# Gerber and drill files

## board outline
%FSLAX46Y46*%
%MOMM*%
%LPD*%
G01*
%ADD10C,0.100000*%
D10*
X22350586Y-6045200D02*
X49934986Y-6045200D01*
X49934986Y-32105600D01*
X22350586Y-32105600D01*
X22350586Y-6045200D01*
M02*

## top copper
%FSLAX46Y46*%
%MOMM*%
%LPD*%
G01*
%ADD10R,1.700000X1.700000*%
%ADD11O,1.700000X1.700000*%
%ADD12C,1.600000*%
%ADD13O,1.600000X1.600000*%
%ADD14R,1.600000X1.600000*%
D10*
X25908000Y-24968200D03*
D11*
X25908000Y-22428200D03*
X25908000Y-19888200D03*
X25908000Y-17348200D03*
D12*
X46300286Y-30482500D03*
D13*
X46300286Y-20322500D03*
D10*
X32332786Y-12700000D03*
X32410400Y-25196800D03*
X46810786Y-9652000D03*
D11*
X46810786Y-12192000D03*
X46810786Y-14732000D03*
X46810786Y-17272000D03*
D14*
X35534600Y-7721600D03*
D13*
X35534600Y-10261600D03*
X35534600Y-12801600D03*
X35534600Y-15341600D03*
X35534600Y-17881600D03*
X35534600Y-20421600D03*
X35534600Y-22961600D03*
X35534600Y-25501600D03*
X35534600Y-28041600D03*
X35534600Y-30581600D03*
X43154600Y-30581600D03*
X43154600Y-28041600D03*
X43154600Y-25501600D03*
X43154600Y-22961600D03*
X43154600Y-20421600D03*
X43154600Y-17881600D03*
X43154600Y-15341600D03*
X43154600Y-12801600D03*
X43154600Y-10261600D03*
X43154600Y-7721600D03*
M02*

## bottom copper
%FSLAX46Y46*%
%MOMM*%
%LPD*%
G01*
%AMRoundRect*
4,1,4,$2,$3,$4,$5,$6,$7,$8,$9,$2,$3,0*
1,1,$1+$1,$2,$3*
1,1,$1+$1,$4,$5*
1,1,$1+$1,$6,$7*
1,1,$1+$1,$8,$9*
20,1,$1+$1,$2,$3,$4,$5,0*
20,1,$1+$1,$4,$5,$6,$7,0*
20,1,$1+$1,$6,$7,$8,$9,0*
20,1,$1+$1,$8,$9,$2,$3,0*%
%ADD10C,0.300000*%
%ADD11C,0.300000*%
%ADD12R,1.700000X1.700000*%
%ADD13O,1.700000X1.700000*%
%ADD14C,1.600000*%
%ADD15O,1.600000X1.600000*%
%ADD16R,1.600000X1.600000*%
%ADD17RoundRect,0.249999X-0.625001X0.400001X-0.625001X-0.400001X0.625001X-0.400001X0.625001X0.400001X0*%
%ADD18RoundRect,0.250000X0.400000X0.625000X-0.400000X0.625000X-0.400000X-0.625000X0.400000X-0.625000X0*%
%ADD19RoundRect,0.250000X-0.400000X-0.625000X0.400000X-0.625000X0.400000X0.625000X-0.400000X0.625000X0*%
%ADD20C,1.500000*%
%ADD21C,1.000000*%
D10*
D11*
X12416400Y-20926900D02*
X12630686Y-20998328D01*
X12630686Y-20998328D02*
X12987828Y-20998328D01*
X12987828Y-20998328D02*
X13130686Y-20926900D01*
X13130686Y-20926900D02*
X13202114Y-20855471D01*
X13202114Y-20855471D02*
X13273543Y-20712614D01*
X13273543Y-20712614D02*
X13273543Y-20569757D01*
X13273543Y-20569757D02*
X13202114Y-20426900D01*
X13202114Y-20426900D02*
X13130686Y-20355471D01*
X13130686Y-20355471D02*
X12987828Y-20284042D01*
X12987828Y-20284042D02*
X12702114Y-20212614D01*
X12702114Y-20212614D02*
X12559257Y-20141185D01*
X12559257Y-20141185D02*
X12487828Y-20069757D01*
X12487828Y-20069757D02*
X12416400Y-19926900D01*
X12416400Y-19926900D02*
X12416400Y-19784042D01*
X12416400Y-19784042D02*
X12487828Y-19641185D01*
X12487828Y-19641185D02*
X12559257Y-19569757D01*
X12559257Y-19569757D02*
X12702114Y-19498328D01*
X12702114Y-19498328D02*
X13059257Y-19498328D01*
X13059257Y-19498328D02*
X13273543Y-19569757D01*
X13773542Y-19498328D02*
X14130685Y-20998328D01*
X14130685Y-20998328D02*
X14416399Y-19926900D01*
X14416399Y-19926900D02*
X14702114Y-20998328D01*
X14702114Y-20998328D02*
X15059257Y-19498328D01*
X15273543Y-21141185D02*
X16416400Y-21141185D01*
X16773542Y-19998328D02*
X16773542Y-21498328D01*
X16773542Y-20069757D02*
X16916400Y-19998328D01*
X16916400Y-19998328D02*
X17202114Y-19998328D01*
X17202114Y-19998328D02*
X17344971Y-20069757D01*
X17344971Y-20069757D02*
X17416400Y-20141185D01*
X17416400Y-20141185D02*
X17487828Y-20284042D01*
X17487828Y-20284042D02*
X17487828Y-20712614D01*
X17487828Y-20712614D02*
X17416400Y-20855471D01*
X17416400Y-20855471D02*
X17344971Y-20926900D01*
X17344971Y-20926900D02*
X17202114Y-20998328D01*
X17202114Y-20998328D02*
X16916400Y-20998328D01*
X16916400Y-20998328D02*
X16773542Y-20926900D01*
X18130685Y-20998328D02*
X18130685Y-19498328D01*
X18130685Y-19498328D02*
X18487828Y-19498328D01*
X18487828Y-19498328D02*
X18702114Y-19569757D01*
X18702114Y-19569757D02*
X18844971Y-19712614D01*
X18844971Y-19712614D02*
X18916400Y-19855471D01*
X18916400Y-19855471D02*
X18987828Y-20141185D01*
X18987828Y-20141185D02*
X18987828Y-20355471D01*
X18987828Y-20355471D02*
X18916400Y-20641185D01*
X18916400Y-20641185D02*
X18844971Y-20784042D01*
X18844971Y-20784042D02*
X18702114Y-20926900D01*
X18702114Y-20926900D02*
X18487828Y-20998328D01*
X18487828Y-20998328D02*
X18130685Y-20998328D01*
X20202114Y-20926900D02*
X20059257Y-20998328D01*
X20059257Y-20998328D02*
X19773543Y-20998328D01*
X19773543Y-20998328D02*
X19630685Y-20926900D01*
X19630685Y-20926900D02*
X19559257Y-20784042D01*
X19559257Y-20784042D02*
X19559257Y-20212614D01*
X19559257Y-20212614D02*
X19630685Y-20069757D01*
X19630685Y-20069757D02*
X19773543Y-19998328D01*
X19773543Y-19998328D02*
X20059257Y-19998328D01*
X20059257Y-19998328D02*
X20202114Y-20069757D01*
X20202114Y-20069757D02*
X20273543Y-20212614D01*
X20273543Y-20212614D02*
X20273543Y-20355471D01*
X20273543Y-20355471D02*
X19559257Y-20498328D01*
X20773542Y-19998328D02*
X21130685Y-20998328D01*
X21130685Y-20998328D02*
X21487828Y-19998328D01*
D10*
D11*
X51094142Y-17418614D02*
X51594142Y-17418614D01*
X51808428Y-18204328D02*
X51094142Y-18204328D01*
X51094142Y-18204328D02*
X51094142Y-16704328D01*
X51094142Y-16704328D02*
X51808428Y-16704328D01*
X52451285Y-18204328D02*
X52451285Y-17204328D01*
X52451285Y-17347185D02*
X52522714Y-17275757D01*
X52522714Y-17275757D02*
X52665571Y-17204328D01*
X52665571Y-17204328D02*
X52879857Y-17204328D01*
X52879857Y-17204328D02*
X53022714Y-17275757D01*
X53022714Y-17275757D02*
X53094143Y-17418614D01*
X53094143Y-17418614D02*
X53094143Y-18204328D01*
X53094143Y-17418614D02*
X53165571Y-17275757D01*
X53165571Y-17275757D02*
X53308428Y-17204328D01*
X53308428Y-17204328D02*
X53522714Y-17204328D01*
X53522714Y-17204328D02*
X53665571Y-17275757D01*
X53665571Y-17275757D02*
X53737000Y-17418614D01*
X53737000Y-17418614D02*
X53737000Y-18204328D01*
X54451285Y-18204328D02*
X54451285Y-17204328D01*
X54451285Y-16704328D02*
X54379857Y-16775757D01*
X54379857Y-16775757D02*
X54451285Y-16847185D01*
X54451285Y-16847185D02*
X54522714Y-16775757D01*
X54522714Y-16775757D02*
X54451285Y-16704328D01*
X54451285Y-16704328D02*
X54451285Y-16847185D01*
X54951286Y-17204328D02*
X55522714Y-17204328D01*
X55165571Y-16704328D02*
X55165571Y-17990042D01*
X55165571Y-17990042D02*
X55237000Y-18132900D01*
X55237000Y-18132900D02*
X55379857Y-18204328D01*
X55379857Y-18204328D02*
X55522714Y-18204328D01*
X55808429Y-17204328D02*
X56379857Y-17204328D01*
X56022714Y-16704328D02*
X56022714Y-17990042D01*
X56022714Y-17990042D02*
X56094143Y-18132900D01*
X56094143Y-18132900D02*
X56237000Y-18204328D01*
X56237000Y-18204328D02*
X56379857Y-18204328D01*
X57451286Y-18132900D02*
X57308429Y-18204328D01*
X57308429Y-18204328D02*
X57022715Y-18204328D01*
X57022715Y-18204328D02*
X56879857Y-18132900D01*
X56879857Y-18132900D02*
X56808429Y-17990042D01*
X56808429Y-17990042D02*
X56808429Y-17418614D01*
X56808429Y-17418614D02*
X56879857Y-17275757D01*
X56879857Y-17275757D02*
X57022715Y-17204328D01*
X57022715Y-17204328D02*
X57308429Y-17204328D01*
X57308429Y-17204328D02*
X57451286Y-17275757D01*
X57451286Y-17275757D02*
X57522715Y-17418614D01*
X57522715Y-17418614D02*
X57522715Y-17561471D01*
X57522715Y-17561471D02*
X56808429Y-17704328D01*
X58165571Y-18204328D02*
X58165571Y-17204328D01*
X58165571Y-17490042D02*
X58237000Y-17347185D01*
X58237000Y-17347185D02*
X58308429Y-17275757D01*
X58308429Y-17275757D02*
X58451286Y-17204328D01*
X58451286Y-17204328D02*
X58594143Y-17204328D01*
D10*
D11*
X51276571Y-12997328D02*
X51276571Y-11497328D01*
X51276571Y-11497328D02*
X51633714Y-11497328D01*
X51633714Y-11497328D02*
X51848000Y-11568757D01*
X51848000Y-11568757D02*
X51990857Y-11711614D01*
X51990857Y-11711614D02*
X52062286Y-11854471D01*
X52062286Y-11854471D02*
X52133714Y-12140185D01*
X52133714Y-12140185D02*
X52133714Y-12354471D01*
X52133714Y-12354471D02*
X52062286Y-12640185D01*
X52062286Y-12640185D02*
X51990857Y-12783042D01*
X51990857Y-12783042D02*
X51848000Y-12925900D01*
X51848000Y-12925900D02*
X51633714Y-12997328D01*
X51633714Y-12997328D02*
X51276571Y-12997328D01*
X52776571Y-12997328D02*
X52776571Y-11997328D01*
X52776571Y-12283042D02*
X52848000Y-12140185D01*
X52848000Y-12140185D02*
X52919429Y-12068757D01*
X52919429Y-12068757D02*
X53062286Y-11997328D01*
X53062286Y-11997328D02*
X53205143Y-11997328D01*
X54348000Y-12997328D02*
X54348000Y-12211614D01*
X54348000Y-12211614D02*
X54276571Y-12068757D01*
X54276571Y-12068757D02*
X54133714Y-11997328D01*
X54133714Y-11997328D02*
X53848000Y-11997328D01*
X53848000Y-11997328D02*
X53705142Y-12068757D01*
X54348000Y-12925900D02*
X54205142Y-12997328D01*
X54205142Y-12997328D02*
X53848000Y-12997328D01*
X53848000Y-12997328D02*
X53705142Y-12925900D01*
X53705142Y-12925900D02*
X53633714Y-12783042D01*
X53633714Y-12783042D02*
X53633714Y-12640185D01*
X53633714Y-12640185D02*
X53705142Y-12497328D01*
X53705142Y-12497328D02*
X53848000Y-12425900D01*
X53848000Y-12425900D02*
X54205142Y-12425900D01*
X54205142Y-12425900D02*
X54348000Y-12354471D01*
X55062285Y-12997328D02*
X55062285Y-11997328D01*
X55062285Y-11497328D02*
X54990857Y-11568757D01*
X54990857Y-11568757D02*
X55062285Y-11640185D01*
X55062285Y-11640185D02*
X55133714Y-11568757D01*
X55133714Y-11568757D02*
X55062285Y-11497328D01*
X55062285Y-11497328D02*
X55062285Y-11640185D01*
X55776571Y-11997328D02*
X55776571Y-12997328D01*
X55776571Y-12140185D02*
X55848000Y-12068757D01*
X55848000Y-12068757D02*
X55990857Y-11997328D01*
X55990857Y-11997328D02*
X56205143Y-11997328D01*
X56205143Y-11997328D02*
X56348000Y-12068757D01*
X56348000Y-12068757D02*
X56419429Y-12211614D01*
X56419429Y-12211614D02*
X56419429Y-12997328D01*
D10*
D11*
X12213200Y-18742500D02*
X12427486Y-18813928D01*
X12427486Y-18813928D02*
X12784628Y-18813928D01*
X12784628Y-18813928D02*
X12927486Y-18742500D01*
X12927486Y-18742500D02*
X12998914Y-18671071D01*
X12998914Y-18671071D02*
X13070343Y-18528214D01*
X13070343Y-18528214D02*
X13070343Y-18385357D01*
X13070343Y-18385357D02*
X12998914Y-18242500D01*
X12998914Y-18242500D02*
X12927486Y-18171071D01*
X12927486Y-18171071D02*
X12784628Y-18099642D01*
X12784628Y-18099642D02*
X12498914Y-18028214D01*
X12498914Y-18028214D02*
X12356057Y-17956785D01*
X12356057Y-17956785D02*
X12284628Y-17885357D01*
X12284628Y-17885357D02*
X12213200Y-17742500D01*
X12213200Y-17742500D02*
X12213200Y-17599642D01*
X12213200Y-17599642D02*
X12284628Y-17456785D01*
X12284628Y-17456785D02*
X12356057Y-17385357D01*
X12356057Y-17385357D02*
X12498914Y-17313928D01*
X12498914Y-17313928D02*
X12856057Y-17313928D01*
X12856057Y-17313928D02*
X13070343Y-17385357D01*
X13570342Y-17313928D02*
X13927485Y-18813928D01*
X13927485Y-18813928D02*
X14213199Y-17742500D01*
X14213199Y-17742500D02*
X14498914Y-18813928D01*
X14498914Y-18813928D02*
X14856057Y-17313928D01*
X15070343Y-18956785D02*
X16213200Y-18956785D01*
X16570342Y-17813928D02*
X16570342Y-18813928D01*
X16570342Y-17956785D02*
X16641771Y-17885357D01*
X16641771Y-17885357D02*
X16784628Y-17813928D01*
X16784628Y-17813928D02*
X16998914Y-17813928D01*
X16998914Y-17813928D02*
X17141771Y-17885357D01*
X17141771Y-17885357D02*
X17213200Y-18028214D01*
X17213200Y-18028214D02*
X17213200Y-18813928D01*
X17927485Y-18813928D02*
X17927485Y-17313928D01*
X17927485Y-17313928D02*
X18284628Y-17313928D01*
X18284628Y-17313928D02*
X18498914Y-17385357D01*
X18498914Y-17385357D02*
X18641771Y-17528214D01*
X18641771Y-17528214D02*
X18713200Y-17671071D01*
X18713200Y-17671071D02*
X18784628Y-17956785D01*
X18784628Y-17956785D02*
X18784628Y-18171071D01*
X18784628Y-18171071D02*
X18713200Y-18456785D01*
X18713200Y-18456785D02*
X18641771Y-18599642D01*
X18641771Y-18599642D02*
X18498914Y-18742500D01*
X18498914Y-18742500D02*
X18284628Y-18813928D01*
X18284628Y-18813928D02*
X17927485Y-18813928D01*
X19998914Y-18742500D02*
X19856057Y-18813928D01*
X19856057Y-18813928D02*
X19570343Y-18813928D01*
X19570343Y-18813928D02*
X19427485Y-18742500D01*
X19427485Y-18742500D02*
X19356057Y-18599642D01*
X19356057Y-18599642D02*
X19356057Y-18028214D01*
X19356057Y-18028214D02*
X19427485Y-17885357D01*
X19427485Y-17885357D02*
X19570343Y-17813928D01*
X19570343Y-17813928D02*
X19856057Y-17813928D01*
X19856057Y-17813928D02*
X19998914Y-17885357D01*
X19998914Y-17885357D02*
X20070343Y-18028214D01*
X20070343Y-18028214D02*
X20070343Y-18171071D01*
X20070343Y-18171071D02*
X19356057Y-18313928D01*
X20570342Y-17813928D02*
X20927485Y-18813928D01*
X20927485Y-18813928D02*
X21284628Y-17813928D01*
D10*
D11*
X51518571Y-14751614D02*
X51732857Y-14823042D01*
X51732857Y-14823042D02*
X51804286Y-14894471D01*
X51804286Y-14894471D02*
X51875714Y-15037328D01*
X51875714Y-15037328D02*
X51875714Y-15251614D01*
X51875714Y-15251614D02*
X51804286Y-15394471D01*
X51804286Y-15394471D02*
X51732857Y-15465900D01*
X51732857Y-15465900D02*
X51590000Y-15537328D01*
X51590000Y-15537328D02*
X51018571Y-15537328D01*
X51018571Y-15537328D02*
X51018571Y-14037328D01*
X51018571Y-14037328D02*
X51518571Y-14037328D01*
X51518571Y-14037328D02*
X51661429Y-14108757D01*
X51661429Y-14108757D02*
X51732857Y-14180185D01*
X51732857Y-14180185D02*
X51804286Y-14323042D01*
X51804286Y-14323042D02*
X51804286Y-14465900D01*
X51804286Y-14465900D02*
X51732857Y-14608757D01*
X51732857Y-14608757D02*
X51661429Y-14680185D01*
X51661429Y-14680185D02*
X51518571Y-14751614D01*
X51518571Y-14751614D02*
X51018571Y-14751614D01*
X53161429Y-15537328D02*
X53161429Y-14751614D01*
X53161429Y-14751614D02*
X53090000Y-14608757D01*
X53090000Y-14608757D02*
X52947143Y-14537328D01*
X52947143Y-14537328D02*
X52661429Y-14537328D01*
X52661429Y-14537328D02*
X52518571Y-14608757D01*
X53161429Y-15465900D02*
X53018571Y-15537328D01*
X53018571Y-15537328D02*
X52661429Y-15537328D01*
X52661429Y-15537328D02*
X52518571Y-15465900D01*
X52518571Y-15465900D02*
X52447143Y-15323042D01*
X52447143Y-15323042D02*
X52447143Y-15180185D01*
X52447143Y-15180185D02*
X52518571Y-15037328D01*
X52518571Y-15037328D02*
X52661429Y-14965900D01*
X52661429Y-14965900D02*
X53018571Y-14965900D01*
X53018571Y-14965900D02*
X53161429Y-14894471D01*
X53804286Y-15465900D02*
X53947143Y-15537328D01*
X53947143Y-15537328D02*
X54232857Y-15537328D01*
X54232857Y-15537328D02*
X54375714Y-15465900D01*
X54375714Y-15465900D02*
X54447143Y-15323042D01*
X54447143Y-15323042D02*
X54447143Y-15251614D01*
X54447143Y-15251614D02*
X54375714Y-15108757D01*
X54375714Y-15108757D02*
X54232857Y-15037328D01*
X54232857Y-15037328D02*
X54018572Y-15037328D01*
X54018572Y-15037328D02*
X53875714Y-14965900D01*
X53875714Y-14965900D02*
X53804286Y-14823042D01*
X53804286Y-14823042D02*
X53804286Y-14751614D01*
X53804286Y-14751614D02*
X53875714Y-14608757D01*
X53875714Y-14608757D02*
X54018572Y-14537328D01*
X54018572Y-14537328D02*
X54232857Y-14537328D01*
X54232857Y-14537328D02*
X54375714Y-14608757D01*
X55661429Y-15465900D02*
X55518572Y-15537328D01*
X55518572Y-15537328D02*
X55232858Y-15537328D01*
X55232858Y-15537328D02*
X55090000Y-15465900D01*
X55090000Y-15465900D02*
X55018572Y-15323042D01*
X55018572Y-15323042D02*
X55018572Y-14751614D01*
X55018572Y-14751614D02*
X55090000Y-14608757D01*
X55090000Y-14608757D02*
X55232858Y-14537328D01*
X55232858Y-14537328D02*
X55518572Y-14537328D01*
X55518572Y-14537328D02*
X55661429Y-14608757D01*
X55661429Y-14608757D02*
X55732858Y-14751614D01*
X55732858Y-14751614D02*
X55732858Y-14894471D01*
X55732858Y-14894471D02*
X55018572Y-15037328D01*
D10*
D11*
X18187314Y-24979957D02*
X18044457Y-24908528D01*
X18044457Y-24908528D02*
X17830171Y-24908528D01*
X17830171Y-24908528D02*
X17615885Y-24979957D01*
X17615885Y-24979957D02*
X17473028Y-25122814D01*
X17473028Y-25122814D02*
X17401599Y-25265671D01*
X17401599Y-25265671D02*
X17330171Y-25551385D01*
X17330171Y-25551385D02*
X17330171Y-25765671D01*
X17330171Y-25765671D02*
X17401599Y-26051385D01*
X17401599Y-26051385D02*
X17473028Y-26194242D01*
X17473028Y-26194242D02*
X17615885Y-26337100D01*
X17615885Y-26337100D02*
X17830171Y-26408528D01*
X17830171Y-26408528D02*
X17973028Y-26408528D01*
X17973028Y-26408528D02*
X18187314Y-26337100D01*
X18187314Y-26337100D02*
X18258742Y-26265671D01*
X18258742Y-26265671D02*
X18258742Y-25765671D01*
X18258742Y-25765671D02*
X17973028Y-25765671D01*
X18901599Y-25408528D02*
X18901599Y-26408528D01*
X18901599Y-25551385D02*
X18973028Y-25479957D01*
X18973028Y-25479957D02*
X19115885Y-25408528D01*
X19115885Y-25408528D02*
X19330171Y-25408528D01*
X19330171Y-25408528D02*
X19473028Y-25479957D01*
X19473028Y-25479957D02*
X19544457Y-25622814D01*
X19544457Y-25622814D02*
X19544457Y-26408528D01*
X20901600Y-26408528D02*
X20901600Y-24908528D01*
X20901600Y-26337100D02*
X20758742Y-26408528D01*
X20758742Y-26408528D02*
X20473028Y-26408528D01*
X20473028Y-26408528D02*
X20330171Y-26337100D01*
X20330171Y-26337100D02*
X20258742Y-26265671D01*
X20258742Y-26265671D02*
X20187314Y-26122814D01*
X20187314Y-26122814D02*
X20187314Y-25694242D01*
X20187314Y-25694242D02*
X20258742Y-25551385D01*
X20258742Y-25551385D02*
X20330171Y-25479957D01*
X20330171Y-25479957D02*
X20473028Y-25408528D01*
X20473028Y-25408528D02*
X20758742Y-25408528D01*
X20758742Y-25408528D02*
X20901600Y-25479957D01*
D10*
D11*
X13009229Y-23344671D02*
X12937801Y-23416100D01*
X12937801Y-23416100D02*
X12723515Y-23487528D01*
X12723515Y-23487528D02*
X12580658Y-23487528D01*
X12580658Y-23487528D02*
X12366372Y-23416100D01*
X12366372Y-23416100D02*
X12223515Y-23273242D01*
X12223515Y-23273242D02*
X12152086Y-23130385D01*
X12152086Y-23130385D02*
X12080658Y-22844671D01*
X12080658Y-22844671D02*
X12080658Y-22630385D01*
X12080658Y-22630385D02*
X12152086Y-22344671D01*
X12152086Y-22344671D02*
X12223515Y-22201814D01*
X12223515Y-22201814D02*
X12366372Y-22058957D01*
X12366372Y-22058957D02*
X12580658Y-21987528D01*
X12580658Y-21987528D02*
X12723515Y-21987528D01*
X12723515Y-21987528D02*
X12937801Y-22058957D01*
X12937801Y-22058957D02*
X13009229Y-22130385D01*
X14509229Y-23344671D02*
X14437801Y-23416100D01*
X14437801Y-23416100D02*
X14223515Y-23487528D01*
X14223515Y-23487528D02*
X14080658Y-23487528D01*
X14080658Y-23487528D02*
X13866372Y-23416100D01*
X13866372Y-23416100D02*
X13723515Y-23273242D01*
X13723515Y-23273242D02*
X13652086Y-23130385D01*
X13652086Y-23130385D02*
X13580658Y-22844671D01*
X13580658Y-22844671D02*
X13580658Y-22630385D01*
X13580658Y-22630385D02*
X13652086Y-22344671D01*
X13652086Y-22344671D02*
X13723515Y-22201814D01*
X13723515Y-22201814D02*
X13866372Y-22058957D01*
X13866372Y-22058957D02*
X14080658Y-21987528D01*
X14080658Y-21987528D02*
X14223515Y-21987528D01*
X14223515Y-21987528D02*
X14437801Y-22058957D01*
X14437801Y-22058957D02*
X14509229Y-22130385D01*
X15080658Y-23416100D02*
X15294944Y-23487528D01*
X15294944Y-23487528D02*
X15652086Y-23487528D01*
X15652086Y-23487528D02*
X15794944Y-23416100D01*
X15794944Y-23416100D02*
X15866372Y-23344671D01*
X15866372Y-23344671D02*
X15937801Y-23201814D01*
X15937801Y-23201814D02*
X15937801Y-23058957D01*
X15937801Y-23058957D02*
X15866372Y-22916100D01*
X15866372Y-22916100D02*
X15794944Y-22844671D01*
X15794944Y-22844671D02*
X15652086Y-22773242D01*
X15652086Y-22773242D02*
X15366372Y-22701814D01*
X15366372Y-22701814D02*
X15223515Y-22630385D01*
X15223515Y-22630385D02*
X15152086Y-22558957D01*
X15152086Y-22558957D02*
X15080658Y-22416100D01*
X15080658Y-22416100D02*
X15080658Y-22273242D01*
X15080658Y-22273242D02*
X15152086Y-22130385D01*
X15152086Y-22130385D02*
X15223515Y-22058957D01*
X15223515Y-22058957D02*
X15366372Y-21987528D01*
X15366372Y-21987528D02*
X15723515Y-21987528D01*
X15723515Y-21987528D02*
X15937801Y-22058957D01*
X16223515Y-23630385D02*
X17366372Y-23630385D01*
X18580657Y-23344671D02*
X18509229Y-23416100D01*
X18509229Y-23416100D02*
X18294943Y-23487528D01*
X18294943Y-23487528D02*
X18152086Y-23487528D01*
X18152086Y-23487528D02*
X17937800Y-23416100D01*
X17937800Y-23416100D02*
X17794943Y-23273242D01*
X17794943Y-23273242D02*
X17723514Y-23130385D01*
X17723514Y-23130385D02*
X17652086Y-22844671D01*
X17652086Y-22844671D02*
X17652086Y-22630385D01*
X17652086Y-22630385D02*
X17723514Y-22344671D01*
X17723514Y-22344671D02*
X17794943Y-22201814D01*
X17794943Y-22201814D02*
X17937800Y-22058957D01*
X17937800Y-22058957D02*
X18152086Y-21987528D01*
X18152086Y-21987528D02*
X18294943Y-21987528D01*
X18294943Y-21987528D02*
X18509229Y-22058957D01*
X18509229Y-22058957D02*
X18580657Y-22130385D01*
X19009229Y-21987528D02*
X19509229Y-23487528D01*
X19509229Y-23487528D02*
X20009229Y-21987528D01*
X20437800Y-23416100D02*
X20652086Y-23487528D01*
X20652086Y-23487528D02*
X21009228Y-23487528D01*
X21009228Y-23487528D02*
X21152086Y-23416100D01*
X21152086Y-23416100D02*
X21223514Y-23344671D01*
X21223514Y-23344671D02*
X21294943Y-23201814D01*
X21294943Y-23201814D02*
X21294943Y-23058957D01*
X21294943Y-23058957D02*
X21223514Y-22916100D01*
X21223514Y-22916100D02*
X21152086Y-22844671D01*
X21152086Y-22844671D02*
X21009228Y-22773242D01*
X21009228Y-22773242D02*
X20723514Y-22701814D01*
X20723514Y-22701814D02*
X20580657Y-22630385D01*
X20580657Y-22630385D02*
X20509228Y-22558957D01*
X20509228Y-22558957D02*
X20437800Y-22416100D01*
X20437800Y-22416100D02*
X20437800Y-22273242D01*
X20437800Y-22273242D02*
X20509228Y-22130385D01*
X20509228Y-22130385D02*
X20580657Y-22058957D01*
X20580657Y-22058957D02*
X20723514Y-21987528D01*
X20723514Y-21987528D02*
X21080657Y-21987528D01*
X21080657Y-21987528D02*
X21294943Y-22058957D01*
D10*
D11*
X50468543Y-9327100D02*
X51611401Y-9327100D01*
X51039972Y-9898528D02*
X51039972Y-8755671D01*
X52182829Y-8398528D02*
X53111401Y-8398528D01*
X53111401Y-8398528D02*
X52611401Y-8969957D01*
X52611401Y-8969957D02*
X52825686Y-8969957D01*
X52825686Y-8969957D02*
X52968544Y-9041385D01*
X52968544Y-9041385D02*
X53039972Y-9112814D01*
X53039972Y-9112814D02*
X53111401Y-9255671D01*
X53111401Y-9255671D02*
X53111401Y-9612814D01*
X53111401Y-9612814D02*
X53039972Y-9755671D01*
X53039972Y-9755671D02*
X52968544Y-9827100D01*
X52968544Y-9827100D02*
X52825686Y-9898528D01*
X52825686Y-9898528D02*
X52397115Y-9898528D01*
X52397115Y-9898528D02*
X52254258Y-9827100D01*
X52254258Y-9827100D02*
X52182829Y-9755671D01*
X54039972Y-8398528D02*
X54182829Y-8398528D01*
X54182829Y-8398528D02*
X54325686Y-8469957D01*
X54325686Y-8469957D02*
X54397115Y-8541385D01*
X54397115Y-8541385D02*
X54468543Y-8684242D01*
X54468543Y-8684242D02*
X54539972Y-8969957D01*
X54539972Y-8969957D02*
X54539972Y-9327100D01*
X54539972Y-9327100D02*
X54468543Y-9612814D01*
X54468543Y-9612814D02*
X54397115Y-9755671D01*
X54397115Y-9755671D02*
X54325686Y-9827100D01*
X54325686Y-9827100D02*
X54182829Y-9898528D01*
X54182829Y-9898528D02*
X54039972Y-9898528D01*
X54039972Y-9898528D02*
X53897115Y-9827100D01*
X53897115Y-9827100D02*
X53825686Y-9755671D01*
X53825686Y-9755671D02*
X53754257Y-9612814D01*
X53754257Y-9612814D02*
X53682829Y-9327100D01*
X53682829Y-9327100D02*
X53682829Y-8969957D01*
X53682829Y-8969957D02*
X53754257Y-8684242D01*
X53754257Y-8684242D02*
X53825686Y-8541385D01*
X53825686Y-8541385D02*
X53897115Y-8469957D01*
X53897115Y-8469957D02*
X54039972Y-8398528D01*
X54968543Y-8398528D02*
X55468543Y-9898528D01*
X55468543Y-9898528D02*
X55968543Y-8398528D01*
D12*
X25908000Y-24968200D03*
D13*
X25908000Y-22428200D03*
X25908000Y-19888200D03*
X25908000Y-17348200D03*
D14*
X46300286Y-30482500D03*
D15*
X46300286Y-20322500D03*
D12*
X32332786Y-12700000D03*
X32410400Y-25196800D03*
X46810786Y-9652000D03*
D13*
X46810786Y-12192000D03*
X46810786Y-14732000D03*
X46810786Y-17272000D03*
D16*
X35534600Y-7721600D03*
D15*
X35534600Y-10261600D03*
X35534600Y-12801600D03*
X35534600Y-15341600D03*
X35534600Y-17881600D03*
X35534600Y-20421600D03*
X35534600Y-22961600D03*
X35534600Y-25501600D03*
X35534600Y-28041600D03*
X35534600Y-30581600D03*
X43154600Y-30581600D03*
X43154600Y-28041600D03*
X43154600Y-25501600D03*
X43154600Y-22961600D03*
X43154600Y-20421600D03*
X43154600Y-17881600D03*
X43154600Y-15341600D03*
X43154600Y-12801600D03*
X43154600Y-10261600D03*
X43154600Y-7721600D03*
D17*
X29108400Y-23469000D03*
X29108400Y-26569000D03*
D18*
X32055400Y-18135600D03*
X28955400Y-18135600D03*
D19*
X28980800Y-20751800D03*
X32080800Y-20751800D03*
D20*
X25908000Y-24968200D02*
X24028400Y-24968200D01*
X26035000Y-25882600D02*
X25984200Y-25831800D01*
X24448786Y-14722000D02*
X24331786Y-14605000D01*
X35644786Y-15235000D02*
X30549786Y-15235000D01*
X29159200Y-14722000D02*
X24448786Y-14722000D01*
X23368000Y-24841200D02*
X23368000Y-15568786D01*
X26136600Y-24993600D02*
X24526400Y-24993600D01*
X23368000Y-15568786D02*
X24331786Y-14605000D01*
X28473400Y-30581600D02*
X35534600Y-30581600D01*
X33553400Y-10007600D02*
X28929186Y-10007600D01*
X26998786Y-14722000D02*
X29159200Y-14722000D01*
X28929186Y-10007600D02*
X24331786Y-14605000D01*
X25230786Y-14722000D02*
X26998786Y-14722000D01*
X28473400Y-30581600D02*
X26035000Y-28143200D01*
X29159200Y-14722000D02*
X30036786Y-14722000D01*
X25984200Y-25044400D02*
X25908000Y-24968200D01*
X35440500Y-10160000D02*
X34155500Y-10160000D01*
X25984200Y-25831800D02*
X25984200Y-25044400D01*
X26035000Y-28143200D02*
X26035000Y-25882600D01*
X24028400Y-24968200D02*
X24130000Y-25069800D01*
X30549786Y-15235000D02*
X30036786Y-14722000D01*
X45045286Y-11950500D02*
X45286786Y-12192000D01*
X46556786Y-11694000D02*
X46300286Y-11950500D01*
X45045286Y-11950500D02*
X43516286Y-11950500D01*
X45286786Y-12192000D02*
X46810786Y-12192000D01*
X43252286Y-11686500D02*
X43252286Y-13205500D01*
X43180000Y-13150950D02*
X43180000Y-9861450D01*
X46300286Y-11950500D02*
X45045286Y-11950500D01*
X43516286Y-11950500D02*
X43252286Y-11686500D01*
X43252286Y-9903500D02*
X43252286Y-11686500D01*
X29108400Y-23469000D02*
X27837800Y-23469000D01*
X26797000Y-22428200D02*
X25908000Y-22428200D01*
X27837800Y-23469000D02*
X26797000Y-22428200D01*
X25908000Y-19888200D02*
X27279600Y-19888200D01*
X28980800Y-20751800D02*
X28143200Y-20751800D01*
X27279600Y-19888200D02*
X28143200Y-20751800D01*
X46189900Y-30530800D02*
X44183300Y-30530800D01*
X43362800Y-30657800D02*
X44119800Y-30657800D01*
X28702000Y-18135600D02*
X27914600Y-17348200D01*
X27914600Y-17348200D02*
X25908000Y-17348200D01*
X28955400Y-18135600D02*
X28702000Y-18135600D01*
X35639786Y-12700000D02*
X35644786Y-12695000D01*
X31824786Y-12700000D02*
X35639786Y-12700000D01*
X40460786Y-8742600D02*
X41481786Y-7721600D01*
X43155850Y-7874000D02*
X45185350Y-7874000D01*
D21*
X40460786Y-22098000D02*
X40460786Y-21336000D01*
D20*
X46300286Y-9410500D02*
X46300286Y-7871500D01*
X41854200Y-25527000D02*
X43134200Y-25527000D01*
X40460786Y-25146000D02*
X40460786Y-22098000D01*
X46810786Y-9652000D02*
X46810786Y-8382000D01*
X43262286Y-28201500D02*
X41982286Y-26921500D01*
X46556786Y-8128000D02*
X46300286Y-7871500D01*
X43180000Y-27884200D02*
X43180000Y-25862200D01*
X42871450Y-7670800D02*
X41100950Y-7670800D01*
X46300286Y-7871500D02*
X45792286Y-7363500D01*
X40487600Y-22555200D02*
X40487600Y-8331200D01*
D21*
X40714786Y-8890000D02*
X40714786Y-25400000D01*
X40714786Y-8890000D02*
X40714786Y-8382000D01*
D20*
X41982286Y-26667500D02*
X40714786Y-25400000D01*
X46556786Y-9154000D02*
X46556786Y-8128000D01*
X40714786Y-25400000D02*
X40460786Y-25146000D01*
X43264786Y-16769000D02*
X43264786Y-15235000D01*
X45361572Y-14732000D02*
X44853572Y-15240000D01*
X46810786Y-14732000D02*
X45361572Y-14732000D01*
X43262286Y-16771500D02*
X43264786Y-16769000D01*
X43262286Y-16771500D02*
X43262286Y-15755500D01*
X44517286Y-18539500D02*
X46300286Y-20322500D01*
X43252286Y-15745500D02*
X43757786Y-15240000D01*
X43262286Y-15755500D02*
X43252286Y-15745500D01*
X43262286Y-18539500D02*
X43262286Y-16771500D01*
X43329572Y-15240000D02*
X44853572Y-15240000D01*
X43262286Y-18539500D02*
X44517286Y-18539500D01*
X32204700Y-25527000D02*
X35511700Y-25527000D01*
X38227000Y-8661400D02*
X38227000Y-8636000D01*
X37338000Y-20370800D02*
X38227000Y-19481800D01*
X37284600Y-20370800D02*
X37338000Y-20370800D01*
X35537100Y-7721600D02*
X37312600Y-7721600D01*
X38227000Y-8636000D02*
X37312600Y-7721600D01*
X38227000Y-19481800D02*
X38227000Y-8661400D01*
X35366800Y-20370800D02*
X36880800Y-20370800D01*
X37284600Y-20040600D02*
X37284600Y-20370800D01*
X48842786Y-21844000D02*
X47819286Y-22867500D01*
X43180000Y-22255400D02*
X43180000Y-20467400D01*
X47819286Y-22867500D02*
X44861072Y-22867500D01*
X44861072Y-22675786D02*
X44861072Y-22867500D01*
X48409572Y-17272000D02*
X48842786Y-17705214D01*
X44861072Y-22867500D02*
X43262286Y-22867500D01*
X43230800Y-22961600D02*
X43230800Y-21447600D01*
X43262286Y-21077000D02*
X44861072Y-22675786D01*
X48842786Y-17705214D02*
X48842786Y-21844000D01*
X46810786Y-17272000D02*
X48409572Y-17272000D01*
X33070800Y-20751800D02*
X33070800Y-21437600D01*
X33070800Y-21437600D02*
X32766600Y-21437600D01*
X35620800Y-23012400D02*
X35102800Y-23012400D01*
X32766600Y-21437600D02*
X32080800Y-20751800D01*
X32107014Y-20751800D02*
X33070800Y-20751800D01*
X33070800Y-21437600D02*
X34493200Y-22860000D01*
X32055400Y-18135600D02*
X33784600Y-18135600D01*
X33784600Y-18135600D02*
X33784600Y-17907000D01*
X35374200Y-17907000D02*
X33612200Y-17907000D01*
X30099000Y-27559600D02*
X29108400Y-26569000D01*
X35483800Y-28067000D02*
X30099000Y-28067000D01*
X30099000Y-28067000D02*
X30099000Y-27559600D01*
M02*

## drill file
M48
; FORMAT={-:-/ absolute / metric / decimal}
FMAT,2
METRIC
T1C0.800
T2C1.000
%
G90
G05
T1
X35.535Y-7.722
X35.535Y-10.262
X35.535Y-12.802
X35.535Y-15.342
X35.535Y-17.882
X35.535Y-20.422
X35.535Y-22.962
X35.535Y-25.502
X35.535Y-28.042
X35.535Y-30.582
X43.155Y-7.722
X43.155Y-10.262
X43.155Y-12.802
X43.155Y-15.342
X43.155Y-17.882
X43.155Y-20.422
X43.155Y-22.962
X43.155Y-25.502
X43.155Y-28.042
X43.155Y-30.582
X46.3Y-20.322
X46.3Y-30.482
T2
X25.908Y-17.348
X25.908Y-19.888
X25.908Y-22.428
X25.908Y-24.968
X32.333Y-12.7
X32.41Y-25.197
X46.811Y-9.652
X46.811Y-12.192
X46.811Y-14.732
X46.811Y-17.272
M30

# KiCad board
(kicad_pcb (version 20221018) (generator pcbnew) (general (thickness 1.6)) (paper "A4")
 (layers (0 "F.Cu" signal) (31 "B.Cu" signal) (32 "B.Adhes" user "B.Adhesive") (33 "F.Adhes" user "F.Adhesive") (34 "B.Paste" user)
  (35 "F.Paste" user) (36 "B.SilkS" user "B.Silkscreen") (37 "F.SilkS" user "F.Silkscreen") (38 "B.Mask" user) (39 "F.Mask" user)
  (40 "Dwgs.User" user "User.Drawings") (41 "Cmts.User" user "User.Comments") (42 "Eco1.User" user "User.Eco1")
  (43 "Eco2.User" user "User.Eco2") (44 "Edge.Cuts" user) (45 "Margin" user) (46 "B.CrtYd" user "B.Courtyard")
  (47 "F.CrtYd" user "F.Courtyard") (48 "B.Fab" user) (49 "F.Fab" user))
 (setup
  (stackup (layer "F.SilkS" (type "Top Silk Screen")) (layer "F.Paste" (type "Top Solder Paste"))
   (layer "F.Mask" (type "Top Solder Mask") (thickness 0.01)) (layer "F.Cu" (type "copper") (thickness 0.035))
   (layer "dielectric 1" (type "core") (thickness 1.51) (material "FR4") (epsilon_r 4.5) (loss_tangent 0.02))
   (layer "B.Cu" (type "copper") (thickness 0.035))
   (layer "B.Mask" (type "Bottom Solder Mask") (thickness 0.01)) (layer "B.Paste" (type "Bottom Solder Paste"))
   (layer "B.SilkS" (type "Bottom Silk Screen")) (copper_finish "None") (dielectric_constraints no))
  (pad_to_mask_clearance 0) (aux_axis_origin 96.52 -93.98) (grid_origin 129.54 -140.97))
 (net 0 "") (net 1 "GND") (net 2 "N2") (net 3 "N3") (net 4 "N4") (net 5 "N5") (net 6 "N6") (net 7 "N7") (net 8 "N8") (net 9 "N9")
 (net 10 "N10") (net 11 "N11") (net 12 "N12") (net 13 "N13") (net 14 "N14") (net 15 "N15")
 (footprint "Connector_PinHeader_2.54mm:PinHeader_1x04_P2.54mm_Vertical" (layer "F.Cu") (at 25.908 24.9682 180)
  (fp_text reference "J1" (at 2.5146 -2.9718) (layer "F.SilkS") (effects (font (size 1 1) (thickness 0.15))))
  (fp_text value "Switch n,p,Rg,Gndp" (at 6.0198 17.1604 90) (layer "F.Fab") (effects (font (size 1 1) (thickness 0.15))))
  (pad "1" thru_hole rect (at 0 0 180) (size 1.7 1.7) (drill 1) (layers "*.Cu" "*.Mask") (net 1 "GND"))
  (pad "2" thru_hole oval (at 0 2.54 180) (size 1.7 1.7) (drill 1) (layers "*.Cu" "*.Mask") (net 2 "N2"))
  (pad "3" thru_hole oval (at 0 5.08 180) (size 1.7 1.7) (drill 1) (layers "*.Cu" "*.Mask") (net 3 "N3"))
  (pad "4" thru_hole oval (at 0 7.62 180) (size 1.7 1.7) (drill 1) (layers "*.Cu" "*.Mask") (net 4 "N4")))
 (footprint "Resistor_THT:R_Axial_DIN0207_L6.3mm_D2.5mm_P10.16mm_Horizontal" (layer "F.Cu") (at 46.300286 30.4825 90)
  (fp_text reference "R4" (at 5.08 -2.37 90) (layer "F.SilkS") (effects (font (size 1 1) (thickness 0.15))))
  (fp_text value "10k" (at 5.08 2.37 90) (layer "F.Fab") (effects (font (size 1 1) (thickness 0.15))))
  (pad "1" thru_hole circle (at 0 0 90) (size 1.6 1.6) (drill 0.8) (layers "*.Cu" "*.Mask") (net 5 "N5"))
  (pad "2" thru_hole oval (at 10.16 0 90) (size 1.6 1.6) (drill 0.8) (layers "*.Cu" "*.Mask") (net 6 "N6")))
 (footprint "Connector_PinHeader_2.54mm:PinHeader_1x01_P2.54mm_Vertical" (layer "F.Cu") (at 32.332786 12.7)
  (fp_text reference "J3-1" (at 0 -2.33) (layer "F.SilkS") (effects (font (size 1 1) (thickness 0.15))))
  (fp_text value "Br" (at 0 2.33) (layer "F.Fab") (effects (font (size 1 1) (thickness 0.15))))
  (pad "1" thru_hole rect (at 0 0) (size 1.7 1.7) (drill 1) (layers "*.Cu" "*.Mask") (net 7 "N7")))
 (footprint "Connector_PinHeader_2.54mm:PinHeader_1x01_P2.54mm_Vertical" (layer "F.Cu") (at 32.4104 25.1968)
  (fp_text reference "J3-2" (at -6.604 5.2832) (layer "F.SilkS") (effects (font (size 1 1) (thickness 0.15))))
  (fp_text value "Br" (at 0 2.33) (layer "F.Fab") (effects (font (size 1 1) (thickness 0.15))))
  (pad "1" thru_hole rect (at 0 0) (size 1.7 1.7) (drill 1) (layers "*.Cu" "*.Mask") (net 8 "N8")))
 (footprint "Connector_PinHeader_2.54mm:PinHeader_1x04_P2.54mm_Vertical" (layer "F.Cu") (at 46.810786 9.652)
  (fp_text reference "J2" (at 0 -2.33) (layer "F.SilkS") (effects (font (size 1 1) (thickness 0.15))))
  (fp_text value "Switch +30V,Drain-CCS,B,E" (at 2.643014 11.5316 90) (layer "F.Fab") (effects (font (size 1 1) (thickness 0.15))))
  (pad "1" thru_hole rect (at 0 0) (size 1.7 1.7) (drill 1) (layers "*.Cu" "*.Mask") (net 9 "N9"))
  (pad "2" thru_hole oval (at 0 2.54) (size 1.7 1.7) (drill 1) (layers "*.Cu" "*.Mask") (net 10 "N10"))
  (pad "3" thru_hole oval (at 0 5.08) (size 1.7 1.7) (drill 1) (layers "*.Cu" "*.Mask") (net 6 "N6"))
  (pad "4" thru_hole oval (at 0 7.62) (size 1.7 1.7) (drill 1) (layers "*.Cu" "*.Mask") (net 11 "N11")))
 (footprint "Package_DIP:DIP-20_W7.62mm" (layer "F.Cu") (at 35.5346 7.7216)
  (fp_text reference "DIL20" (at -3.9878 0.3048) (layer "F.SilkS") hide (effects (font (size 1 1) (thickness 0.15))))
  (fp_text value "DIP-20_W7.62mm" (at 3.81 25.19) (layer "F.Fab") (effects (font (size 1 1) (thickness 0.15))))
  (pad "1" thru_hole rect (at 0 0) (size 1.6 1.6) (drill 0.8) (layers "*.Cu" "*.Mask"))
  (pad "2" thru_hole oval (at 0 2.54) (size 1.6 1.6) (drill 0.8) (layers "*.Cu" "*.Mask"))
  (pad "3" thru_hole oval (at 0 5.08) (size 1.6 1.6) (drill 0.8) (layers "*.Cu" "*.Mask"))
  (pad "4" thru_hole oval (at 0 7.62) (size 1.6 1.6) (drill 0.8) (layers "*.Cu" "*.Mask"))
  (pad "5" thru_hole oval (at 0 10.16) (size 1.6 1.6) (drill 0.8) (layers "*.Cu" "*.Mask"))
  (pad "6" thru_hole oval (at 0 12.7) (size 1.6 1.6) (drill 0.8) (layers "*.Cu" "*.Mask"))
  (pad "7" thru_hole oval (at 0 15.24) (size 1.6 1.6) (drill 0.8) (layers "*.Cu" "*.Mask"))
  (pad "8" thru_hole oval (at 0 17.78) (size 1.6 1.6) (drill 0.8) (layers "*.Cu" "*.Mask"))
  (pad "9" thru_hole oval (at 0 20.32) (size 1.6 1.6) (drill 0.8) (layers "*.Cu" "*.Mask"))
  (pad "10" thru_hole oval (at 0 22.86) (size 1.6 1.6) (drill 0.8) (layers "*.Cu" "*.Mask"))
  (pad "11" thru_hole oval (at 7.62 22.86) (size 1.6 1.6) (drill 0.8) (layers "*.Cu" "*.Mask"))
  (pad "12" thru_hole oval (at 7.62 20.32) (size 1.6 1.6) (drill 0.8) (layers "*.Cu" "*.Mask"))
  (pad "13" thru_hole oval (at 7.62 17.78) (size 1.6 1.6) (drill 0.8) (layers "*.Cu" "*.Mask"))
  (pad "14" thru_hole oval (at 7.62 15.24) (size 1.6 1.6) (drill 0.8) (layers "*.Cu" "*.Mask"))
  (pad "15" thru_hole oval (at 7.62 12.7) (size 1.6 1.6) (drill 0.8) (layers "*.Cu" "*.Mask"))
  (pad "16" thru_hole oval (at 7.62 10.16) (size 1.6 1.6) (drill 0.8) (layers "*.Cu" "*.Mask"))
  (pad "17" thru_hole oval (at 7.62 7.62) (size 1.6 1.6) (drill 0.8) (layers "*.Cu" "*.Mask"))
  (pad "18" thru_hole oval (at 7.62 5.08) (size 1.6 1.6) (drill 0.8) (layers "*.Cu" "*.Mask"))
  (pad "19" thru_hole oval (at 7.62 2.54) (size 1.6 1.6) (drill 0.8) (layers "*.Cu" "*.Mask"))
  (pad "20" thru_hole oval (at 7.62 0) (size 1.6 1.6) (drill 0.8) (layers "*.Cu" "*.Mask")))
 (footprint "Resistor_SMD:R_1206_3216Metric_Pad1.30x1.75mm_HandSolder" (layer "B.Cu") (at 29.1084 25.019 -90)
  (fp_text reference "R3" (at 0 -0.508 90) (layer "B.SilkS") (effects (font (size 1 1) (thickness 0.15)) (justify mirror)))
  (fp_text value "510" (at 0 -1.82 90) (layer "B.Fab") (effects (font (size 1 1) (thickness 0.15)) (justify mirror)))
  (pad "1" smd roundrect (at -1.55 0 270) (size 1.3 1.75) (layers "B.Cu" "B.Paste" "B.Mask") (roundrect_rratio 0.1923069231) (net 2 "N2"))
  (pad "2" smd roundrect (at 1.55 0 270) (size 1.3 1.75) (layers "B.Cu" "B.Paste" "B.Mask") (roundrect_rratio 0.1923069231) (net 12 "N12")))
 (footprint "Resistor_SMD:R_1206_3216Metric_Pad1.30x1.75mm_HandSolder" (layer "B.Cu") (at 30.5054 18.1356 180)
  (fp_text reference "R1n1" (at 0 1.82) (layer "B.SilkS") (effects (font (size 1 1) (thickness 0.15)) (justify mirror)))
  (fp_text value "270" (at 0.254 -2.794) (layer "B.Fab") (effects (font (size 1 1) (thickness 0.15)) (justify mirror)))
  (pad "1" smd roundrect (at -1.55 0 180) (size 1.3 1.75) (layers "B.Cu" "B.Paste" "B.Mask") (roundrect_rratio 0.192308) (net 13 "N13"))
  (pad "2" smd roundrect (at 1.55 0 180) (size 1.3 1.75) (layers "B.Cu" "B.Paste" "B.Mask") (roundrect_rratio 0.192308) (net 4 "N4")))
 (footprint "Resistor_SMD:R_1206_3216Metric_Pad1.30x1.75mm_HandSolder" (layer "B.Cu") (at 30.5308 20.7518)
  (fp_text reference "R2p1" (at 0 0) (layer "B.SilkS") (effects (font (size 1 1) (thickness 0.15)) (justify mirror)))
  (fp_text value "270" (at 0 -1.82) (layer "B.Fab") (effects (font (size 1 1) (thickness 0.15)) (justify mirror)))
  (pad "1" smd roundrect (at -1.55 0) (size 1.3 1.75) (layers "B.Cu" "B.Paste" "B.Mask") (roundrect_rratio 0.192308) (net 3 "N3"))
  (pad "2" smd roundrect (at 1.55 0) (size 1.3 1.75) (layers "B.Cu" "B.Paste" "B.Mask") (roundrect_rratio 0.192308) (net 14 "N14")))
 (gr_rect (start 22.350586 6.0452) (end 49.934986 32.1056) (stroke (width 0.1) (type solid)) (fill none) (layer "Edge.Cuts"))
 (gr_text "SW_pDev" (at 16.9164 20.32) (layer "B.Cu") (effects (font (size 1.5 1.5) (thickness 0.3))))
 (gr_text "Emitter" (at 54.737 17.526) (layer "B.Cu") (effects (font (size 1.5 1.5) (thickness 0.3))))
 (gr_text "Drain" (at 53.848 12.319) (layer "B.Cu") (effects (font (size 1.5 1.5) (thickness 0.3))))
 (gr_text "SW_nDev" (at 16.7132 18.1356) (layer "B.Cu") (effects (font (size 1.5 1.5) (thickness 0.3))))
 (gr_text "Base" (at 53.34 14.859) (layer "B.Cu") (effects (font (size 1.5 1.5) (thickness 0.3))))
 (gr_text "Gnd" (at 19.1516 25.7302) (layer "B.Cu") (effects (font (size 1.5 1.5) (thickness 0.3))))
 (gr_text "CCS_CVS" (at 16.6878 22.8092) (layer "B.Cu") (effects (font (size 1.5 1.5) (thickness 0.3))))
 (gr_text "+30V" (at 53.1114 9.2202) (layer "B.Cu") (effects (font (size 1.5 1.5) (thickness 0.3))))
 (segment (start 25.908 24.9682) (end 24.0284 24.9682) (width 1.5) (layer "B.Cu") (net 1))
 (segment (start 26.035 25.8826) (end 25.9842 25.8318) (width 1.5) (layer "B.Cu") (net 1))
 (segment (start 24.448786 14.722) (end 24.331786 14.605) (width 1.5) (layer "B.Cu") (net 1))
 (segment (start 35.644786 15.235) (end 30.549786 15.235) (width 1.5) (layer "B.Cu") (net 1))
 (segment (start 29.1592 14.722) (end 24.448786 14.722) (width 1.5) (layer "B.Cu") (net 1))
 (segment (start 23.368 24.8412) (end 23.368 15.568786) (width 1.5) (layer "B.Cu") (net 1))
 (segment (start 26.1366 24.9936) (end 24.5264 24.9936) (width 1.5) (layer "B.Cu") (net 1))
 (segment (start 23.368 15.568786) (end 24.331786 14.605) (width 1.5) (layer "B.Cu") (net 1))
 (segment (start 28.4734 30.5816) (end 35.5346 30.5816) (width 1.5) (layer "B.Cu") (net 1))
 (segment (start 33.5534 10.0076) (end 28.929186 10.0076) (width 1.5) (layer "B.Cu") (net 1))
 (segment (start 26.998786 14.722) (end 29.1592 14.722) (width 1.5) (layer "B.Cu") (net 1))
 (segment (start 28.929186 10.0076) (end 24.331786 14.605) (width 1.5) (layer "B.Cu") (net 1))
 (segment (start 25.230786 14.722) (end 26.998786 14.722) (width 1.5) (layer "B.Cu") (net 1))
 (segment (start 28.4734 30.5816) (end 26.035 28.1432) (width 1.5) (layer "B.Cu") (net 1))
 (segment (start 29.1592 14.722) (end 30.036786 14.722) (width 1.5) (layer "B.Cu") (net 1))
 (segment (start 25.9842 25.0444) (end 25.908 24.9682) (width 1.5) (layer "B.Cu") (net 1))
 (segment (start 35.4405 10.16) (end 34.1555 10.16) (width 1.5) (layer "B.Cu") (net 1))
 (segment (start 25.9842 25.8318) (end 25.9842 25.0444) (width 1.5) (layer "B.Cu") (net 1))
 (segment (start 26.035 28.1432) (end 26.035 25.8826) (width 1.5) (layer "B.Cu") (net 1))
 (segment (start 24.0284 24.9682) (end 24.13 25.0698) (width 1.5) (layer "B.Cu") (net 1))
 (segment (start 30.549786 15.235) (end 30.036786 14.722) (width 1.5) (layer "B.Cu") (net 1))
 (segment (start 45.045286 11.9505) (end 45.286786 12.192) (width 1.5) (layer "B.Cu") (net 10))
 (segment (start 46.556786 11.694) (end 46.300286 11.9505) (width 1.5) (layer "B.Cu") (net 10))
 (segment (start 45.045286 11.9505) (end 43.516286 11.9505) (width 1.5) (layer "B.Cu") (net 10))
 (segment (start 45.286786 12.192) (end 46.810786 12.192) (width 1.5) (layer "B.Cu") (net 10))
 (segment (start 43.252286 11.6865) (end 43.252286 13.2055) (width 1.5) (layer "B.Cu") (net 10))
 (segment (start 43.18 13.15095) (end 43.18 9.86145) (width 1.5) (layer "B.Cu") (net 10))
 (segment (start 46.300286 11.9505) (end 45.045286 11.9505) (width 1.5) (layer "B.Cu") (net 10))
 (segment (start 43.516286 11.9505) (end 43.252286 11.6865) (width 1.5) (layer "B.Cu") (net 10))
 (segment (start 43.252286 9.9035) (end 43.252286 11.6865) (width 1.5) (layer "B.Cu") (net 10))
 (segment (start 29.1084 23.469) (end 27.8378 23.469) (width 1.5) (layer "B.Cu") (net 2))
 (segment (start 26.797 22.4282) (end 25.908 22.4282) (width 1.5) (layer "B.Cu") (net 2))
 (segment (start 27.8378 23.469) (end 26.797 22.4282) (width 1.5) (layer "B.Cu") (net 2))
 (segment (start 25.908 19.8882) (end 27.2796 19.8882) (width 1.5) (layer "B.Cu") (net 3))
 (segment (start 28.9808 20.7518) (end 28.1432 20.7518) (width 1.5) (layer "B.Cu") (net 3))
 (segment (start 27.2796 19.8882) (end 28.1432 20.7518) (width 1.5) (layer "B.Cu") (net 3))
 (segment (start 46.1899 30.5308) (end 44.1833 30.5308) (width 1.5) (layer "B.Cu") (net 5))
 (segment (start 43.3628 30.6578) (end 44.1198 30.6578) (width 1.5) (layer "B.Cu") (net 5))
 (segment (start 28.702 18.1356) (end 27.9146 17.3482) (width 1.5) (layer "B.Cu") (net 4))
 (segment (start 27.9146 17.3482) (end 25.908 17.3482) (width 1.5) (layer "B.Cu") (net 4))
 (segment (start 28.9554 18.1356) (end 28.702 18.1356) (width 1.5) (layer "B.Cu") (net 4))
 (segment (start 35.639786 12.7) (end 35.644786 12.695) (width 1.5) (layer "B.Cu") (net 7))
 (segment (start 31.824786 12.7) (end 35.639786 12.7) (width 1.5) (layer "B.Cu") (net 7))
 (segment (start 40.460786 8.7426) (end 41.481786 7.7216) (width 1.5) (layer "B.Cu") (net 9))
 (segment (start 43.15585 7.874) (end 45.18535 7.874) (width 1.5) (layer "B.Cu") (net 9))
 (segment (start 40.460786 22.098) (end 40.460786 21.336) (width 1) (layer "B.Cu") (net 9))
 (segment (start 46.300286 9.4105) (end 46.300286 7.8715) (width 1.5) (layer "B.Cu") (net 9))
 (segment (start 41.8542 25.527) (end 43.1342 25.527) (width 1.5) (layer "B.Cu") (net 9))
 (segment (start 40.460786 25.146) (end 40.460786 22.098) (width 1.5) (layer "B.Cu") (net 9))
 (segment (start 46.810786 9.652) (end 46.810786 8.382) (width 1.5) (layer "B.Cu") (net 9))
 (segment (start 43.262286 28.2015) (end 41.982286 26.9215) (width 1.5) (layer "B.Cu") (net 9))
 (segment (start 46.556786 8.128) (end 46.300286 7.8715) (width 1.5) (layer "B.Cu") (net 9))
 (segment (start 43.18 27.8842) (end 43.18 25.8622) (width 1.5) (layer "B.Cu") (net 9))
 (segment (start 42.87145 7.6708) (end 41.10095 7.6708) (width 1.5) (layer "B.Cu") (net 9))
 (segment (start 46.300286 7.8715) (end 45.792286 7.3635) (width 1.5) (layer "B.Cu") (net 9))
 (segment (start 40.4876 22.5552) (end 40.4876 8.3312) (width 1.5) (layer "B.Cu") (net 9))
 (segment (start 40.714786 8.89) (end 40.714786 25.4) (width 1) (layer "B.Cu") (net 9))
 (segment (start 40.714786 8.89) (end 40.714786 8.382) (width 1) (layer "B.Cu") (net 9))
 (segment (start 41.982286 26.6675) (end 40.714786 25.4) (width 1.5) (layer "B.Cu") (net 9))
 (segment (start 46.556786 9.154) (end 46.556786 8.128) (width 1.5) (layer "B.Cu") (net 9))
 (segment (start 40.714786 25.4) (end 40.460786 25.146) (width 1.5) (layer "B.Cu") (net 9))
 (segment (start 43.264786 16.769) (end 43.264786 15.235) (width 1.5) (layer "B.Cu") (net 6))
 (segment (start 45.361572 14.732) (end 44.853572 15.24) (width 1.5) (layer "B.Cu") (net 6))
 (segment (start 46.810786 14.732) (end 45.361572 14.732) (width 1.5) (layer "B.Cu") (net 6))
 (segment (start 43.262286 16.7715) (end 43.264786 16.769) (width 1.5) (layer "B.Cu") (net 6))
 (segment (start 43.262286 16.7715) (end 43.262286 15.7555) (width 1.5) (layer "B.Cu") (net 6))
 (segment (start 44.517286 18.5395) (end 46.300286 20.3225) (width 1.5) (layer "B.Cu") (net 6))
 (segment (start 43.252286 15.7455) (end 43.757786 15.24) (width 1.5) (layer "B.Cu") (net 6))
 (segment (start 43.262286 15.7555) (end 43.252286 15.7455) (width 1.5) (layer "B.Cu") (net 6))
 (segment (start 43.262286 18.5395) (end 43.262286 16.7715) (width 1.5) (layer "B.Cu") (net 6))
 (segment (start 43.329572 15.24) (end 44.853572 15.24) (width 1.5) (layer "B.Cu") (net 6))
 (segment (start 43.262286 18.5395) (end 44.517286 18.5395) (width 1.5) (layer "B.Cu") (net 6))
 (segment (start 32.2047 25.527) (end 35.5117 25.527) (width 1.5) (layer "B.Cu") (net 8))
 (segment (start 38.227 8.6614) (end 38.227 8.636) (width 1.5) (layer "B.Cu") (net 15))
 (segment (start 37.338 20.3708) (end 38.227 19.4818) (width 1.5) (layer "B.Cu") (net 15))
 (segment (start 37.2846 20.3708) (end 37.338 20.3708) (width 1.5) (layer "B.Cu") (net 15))
 (segment (start 35.5371 7.7216) (end 37.3126 7.7216) (width 1.5) (layer "B.Cu") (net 15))
 (segment (start 38.227 8.636) (end 37.3126 7.7216) (width 1.5) (layer "B.Cu") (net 15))
 (segment (start 38.227 19.4818) (end 38.227 8.6614) (width 1.5) (layer "B.Cu") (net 15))
 (segment (start 35.3668 20.3708) (end 36.8808 20.3708) (width 1.5) (layer "B.Cu") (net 15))
 (segment (start 37.2846 20.0406) (end 37.2846 20.3708) (width 1.5) (layer "B.Cu") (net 15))
 (segment (start 48.842786 21.844) (end 47.819286 22.8675) (width 1.5) (layer "B.Cu") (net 11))
 (segment (start 43.18 22.2554) (end 43.18 20.4674) (width 1.5) (layer "B.Cu") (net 11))
 (segment (start 47.819286 22.8675) (end 44.861072 22.8675) (width 1.5) (layer "B.Cu") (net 11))
 (segment (start 44.861072 22.675786) (end 44.861072 22.8675) (width 1.5) (layer "B.Cu") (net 11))
 (segment (start 48.409572 17.272) (end 48.842786 17.705214) (width 1.5) (layer "B.Cu") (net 11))
 (segment (start 44.861072 22.8675) (end 43.262286 22.8675) (width 1.5) (layer "B.Cu") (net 11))
 (segment (start 43.2308 22.9616) (end 43.2308 21.4476) (width 1.5) (layer "B.Cu") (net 11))
 (segment (start 43.262286 21.077) (end 44.861072 22.675786) (width 1.5) (layer "B.Cu") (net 11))
 (segment (start 48.842786 17.705214) (end 48.842786 21.844) (width 1.5) (layer "B.Cu") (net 11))
 (segment (start 46.810786 17.272) (end 48.409572 17.272) (width 1.5) (layer "B.Cu") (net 11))
 (segment (start 33.0708 20.7518) (end 33.0708 21.4376) (width 1.5) (layer "B.Cu") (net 14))
 (segment (start 33.0708 21.4376) (end 32.7666 21.4376) (width 1.5) (layer "B.Cu") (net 14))
 (segment (start 35.6208 23.0124) (end 35.1028 23.0124) (width 1.5) (layer "B.Cu") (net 14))
 (segment (start 32.7666 21.4376) (end 32.0808 20.7518) (width 1.5) (layer "B.Cu") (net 14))
 (segment (start 32.107014 20.7518) (end 33.0708 20.7518) (width 1.5) (layer "B.Cu") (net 14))
 (segment (start 33.0708 21.4376) (end 34.4932 22.86) (width 1.5) (layer "B.Cu") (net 14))
 (segment (start 32.0554 18.1356) (end 33.7846 18.1356) (width 1.5) (layer "B.Cu") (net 13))
 (segment (start 33.7846 18.1356) (end 33.7846 17.907) (width 1.5) (layer "B.Cu") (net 13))
 (segment (start 35.3742 17.907) (end 33.6122 17.907) (width 1.5) (layer "B.Cu") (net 13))
 (segment (start 30.099 27.5596) (end 29.1084 26.569) (width 1.5) (layer "B.Cu") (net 12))
 (segment (start 35.4838 28.067) (end 30.099 28.067) (width 1.5) (layer "B.Cu") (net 12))
 (segment (start 30.099 28.067) (end 30.099 27.5596) (width 1.5) (layer "B.Cu") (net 12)))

